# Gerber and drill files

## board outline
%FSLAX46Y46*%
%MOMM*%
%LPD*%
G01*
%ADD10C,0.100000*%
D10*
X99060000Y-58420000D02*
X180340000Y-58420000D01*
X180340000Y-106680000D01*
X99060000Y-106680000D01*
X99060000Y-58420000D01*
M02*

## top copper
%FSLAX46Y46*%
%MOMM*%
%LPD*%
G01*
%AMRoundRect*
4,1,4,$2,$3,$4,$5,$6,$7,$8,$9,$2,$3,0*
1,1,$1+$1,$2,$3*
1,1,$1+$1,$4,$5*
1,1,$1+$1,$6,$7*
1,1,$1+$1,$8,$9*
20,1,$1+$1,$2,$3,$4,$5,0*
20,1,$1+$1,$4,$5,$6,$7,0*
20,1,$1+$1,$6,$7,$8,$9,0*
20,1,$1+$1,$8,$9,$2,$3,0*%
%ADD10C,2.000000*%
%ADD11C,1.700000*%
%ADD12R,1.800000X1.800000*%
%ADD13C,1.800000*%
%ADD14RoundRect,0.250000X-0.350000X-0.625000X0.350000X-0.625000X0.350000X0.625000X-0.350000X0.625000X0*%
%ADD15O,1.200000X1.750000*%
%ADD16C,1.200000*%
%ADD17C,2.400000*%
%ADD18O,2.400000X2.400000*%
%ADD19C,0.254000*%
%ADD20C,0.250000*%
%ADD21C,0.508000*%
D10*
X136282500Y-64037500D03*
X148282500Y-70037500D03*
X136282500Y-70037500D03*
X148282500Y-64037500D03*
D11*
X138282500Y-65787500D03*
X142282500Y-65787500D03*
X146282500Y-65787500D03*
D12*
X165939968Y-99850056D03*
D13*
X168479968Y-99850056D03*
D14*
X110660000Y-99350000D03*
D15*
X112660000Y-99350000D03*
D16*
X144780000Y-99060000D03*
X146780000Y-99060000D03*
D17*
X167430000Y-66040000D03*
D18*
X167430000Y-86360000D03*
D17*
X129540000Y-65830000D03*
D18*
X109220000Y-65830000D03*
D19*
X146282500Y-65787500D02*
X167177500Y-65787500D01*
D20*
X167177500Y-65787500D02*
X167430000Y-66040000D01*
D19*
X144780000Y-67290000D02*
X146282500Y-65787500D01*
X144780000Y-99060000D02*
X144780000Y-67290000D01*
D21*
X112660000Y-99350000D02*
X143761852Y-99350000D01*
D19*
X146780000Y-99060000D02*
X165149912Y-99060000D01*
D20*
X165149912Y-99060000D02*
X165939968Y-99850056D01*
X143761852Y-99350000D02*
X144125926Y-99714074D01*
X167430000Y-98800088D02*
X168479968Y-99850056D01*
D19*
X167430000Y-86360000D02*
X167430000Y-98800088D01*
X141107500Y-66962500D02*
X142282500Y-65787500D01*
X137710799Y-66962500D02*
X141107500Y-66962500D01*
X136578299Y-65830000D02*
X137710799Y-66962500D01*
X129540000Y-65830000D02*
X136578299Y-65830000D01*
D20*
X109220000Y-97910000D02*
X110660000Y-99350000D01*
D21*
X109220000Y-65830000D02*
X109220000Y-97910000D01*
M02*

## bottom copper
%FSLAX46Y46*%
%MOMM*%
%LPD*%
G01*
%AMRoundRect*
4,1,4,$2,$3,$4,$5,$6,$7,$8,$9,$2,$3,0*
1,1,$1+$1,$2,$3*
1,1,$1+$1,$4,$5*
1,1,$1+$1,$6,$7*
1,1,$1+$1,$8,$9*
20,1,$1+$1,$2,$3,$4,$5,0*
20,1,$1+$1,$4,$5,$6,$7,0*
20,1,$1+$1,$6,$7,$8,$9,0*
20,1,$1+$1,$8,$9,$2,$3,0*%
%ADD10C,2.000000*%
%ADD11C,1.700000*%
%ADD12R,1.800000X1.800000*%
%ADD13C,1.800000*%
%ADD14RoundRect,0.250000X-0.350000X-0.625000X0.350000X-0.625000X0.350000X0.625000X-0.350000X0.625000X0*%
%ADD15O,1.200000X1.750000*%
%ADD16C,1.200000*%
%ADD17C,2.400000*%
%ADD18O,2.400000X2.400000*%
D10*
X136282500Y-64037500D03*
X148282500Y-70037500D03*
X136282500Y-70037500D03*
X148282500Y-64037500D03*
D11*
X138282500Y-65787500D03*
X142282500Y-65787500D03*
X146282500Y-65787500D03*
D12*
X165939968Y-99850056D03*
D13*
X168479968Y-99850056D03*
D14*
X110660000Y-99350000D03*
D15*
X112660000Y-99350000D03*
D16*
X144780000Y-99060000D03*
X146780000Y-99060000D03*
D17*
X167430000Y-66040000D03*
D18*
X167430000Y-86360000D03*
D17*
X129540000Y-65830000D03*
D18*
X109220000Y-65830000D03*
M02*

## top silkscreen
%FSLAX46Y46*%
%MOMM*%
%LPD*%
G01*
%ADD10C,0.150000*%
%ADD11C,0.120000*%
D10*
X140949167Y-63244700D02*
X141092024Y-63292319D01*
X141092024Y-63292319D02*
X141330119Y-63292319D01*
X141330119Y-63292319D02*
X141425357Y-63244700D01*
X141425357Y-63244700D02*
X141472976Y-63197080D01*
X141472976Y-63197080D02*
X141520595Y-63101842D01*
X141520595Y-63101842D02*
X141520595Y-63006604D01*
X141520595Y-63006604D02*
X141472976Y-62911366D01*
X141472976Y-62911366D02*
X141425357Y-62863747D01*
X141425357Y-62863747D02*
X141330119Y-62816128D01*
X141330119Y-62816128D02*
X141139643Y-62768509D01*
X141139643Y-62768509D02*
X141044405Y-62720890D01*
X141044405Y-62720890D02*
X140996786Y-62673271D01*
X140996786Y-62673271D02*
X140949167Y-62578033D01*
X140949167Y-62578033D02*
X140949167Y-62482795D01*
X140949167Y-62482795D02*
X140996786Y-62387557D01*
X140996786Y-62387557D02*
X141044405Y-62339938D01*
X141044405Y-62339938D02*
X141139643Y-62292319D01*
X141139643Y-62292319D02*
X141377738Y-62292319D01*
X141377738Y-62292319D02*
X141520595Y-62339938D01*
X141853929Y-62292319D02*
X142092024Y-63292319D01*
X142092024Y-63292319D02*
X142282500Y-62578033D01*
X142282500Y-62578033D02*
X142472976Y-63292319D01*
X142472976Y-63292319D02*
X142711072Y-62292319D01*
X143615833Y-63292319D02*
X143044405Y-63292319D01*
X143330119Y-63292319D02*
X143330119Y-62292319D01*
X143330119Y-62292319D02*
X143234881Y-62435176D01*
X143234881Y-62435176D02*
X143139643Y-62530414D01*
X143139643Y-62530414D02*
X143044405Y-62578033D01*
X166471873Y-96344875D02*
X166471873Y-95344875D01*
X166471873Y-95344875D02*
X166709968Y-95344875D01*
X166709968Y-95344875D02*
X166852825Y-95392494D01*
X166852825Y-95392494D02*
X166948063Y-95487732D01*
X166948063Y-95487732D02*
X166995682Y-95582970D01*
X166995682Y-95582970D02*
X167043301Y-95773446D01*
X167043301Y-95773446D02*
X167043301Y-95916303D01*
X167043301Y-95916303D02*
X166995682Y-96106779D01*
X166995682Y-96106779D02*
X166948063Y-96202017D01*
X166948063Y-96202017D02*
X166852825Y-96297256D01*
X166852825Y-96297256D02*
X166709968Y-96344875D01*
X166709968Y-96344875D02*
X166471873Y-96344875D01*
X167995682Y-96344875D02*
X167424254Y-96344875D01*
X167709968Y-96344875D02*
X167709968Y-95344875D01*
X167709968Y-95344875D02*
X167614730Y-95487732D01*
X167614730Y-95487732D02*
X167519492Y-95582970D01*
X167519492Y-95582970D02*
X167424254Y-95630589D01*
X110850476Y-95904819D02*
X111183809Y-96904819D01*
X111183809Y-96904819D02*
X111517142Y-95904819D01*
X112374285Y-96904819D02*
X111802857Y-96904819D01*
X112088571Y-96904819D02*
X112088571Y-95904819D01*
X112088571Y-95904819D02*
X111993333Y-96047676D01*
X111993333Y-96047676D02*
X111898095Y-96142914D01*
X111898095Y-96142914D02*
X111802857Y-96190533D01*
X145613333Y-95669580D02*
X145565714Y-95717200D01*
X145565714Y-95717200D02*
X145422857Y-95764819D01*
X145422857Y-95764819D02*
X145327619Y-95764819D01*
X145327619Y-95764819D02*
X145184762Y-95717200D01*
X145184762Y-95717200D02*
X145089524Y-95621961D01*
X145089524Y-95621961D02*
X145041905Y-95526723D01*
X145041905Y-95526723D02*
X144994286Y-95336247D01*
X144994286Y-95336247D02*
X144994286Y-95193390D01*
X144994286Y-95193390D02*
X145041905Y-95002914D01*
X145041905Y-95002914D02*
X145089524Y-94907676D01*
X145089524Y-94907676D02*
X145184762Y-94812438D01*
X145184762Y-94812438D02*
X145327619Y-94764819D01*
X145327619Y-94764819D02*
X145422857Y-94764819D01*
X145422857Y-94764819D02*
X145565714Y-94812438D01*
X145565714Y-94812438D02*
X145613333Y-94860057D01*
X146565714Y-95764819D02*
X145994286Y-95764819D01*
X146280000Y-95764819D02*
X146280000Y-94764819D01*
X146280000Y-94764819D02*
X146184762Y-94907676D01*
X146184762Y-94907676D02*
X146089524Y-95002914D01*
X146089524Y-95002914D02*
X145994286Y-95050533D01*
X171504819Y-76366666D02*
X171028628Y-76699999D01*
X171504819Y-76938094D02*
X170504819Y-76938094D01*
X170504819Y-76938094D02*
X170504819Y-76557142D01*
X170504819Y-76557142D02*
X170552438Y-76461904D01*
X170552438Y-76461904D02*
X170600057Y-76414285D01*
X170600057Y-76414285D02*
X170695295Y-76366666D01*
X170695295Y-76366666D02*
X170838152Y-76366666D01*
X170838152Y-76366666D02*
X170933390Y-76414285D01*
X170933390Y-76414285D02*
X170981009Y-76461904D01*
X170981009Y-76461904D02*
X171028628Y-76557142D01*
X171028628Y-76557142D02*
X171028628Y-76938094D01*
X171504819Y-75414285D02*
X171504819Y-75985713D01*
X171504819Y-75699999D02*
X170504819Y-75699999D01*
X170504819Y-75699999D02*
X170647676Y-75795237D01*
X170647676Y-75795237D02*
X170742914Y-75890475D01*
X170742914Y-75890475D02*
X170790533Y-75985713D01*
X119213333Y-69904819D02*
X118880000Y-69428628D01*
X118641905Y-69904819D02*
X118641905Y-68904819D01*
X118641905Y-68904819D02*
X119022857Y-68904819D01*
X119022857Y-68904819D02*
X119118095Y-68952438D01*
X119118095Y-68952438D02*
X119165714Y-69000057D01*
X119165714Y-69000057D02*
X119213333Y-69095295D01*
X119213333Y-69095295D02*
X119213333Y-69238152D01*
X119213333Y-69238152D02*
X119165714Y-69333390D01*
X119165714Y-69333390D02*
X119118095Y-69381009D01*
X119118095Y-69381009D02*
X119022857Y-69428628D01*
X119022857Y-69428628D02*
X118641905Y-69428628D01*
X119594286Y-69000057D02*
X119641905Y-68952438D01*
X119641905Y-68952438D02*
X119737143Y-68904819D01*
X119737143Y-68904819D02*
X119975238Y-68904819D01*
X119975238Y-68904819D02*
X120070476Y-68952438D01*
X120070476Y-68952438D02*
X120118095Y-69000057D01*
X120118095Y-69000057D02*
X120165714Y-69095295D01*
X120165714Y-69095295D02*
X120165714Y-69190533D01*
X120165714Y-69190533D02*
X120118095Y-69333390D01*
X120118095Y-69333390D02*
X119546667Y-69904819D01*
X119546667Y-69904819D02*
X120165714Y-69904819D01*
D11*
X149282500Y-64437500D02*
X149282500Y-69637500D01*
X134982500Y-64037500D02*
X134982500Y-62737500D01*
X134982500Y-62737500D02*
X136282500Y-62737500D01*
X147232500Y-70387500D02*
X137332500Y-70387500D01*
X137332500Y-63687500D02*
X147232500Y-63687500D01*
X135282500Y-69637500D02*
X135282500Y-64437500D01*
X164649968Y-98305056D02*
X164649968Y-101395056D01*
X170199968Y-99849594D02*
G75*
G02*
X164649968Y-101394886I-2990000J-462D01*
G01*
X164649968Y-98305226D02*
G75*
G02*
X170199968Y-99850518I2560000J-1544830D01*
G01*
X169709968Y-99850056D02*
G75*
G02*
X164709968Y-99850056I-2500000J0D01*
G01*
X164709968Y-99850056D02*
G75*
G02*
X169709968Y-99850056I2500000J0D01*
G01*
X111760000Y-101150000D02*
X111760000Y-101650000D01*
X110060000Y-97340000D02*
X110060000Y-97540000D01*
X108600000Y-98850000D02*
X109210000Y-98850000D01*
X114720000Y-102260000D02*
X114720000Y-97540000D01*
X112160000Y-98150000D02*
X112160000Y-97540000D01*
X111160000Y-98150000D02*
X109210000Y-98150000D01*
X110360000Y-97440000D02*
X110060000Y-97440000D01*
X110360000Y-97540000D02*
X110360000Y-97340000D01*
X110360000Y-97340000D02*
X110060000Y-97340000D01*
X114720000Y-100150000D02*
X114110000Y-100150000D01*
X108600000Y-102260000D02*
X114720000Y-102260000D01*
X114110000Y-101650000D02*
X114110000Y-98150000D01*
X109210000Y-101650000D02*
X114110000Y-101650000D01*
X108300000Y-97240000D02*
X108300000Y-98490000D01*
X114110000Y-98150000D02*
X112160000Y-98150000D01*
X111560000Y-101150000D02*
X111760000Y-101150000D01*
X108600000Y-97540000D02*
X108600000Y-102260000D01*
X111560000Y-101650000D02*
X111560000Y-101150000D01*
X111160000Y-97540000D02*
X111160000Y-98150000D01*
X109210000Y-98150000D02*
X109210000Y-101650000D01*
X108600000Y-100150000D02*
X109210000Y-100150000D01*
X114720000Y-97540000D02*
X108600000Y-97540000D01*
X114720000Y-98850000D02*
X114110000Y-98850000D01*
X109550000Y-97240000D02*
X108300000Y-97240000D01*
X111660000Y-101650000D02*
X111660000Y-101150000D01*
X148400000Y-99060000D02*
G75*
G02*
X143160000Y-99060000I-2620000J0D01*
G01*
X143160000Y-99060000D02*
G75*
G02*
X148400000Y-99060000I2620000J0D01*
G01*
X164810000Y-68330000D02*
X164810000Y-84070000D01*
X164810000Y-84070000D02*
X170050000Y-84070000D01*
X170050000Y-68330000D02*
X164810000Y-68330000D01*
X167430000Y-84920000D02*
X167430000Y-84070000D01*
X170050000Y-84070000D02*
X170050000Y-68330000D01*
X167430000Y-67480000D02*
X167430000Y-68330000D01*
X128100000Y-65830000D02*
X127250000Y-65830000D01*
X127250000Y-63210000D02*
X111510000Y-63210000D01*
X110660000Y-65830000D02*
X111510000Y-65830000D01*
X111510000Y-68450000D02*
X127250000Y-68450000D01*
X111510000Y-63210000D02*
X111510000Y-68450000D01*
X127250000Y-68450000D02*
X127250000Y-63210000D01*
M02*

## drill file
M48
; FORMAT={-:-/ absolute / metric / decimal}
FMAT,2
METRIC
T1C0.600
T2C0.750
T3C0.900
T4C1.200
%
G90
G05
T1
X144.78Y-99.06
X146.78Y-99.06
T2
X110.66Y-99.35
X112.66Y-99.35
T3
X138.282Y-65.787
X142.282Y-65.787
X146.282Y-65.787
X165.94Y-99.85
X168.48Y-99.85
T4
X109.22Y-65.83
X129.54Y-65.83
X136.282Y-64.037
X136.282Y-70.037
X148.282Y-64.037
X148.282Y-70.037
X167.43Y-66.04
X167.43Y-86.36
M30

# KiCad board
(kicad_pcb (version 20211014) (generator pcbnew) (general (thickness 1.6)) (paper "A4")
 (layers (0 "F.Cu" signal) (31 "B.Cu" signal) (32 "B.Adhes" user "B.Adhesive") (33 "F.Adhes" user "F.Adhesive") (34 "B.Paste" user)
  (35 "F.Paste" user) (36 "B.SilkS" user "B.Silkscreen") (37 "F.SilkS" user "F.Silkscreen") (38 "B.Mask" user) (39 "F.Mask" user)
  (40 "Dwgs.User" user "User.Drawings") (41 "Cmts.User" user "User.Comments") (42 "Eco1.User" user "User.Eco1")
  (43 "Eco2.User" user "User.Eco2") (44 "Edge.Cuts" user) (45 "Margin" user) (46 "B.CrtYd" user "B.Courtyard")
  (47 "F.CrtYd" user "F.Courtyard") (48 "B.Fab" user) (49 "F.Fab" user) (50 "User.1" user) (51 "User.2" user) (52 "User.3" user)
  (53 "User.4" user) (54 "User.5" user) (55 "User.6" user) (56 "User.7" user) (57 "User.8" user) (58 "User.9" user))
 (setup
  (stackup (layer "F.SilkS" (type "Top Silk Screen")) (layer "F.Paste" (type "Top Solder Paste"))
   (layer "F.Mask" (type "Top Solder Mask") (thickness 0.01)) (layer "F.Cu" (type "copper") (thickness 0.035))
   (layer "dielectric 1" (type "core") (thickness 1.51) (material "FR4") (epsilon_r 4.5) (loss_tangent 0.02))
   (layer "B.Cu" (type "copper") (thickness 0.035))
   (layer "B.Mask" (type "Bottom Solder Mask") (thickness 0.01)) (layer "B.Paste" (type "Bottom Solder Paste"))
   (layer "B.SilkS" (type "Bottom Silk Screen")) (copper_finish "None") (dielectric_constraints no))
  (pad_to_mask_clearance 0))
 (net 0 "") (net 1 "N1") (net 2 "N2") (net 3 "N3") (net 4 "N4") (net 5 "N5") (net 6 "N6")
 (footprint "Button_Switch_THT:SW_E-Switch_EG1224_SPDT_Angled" (layer "F.Cu") (at 138.2825 65.7875)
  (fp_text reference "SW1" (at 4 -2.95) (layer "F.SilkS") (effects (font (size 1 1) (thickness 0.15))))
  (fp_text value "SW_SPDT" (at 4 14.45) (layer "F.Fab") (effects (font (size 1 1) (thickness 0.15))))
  (fp_line (start 11 -1.35) (end 11 3.85) (layer "F.SilkS") (width 0.12))
  (fp_line (start -3.3 -1.75) (end -3.3 -3.05) (layer "F.SilkS") (width 0.12))
  (fp_line (start -3.3 -3.05) (end -2 -3.05) (layer "F.SilkS") (width 0.12))
  (fp_line (start 8.95 4.6) (end -0.95 4.6) (layer "F.SilkS") (width 0.12))
  (fp_line (start -0.95 -2.1) (end 8.95 -2.1) (layer "F.SilkS") (width 0.12))
  (fp_line (start -3 3.85) (end -3 -1.35) (layer "F.SilkS") (width 0.12))
  (pad "" thru_hole circle (at -2 -1.75) (size 2 2) (drill 1.2) (layers *.Cu *.Mask))
  (pad "" thru_hole circle (at 10 4.25) (size 2 2) (drill 1.2) (layers *.Cu *.Mask))
  (pad "" thru_hole circle (at -2 4.25) (size 2 2) (drill 1.2) (layers *.Cu *.Mask))
  (pad "" thru_hole circle (at 10 -1.75) (size 2 2) (drill 1.2) (layers *.Cu *.Mask))
  (pad "1" thru_hole circle (at 0 0) (size 1.7 1.7) (drill 0.9) (layers *.Cu *.Mask) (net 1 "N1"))
  (pad "2" thru_hole circle (at 4 0) (size 1.7 1.7) (drill 0.9) (layers *.Cu *.Mask) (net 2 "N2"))
  (pad "3" thru_hole circle (at 8 0) (size 1.7 1.7) (drill 0.9) (layers *.Cu *.Mask) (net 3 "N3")))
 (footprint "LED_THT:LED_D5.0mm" (layer "F.Cu") (at 165.939968 99.850056)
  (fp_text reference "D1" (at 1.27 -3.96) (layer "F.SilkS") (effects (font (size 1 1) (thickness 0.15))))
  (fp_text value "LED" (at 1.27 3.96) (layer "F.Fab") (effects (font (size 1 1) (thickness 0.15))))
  (fp_line (start -1.29 -1.545) (end -1.29 1.545) (layer "F.SilkS") (width 0.12))
  (fp_arc (start 4.26 -0.000462) (mid 2.072002 2.880433) (end -1.29 1.54483) (layer "F.SilkS") (width 0.12))
  (fp_arc (start -1.29 -1.54483) (mid 2.072002 -2.880433) (end 4.26 0.000462) (layer "F.SilkS") (width 0.12))
  (fp_circle (center 1.27 0) (end 3.77 0) (layer "F.SilkS") (width 0.12) (fill none))
  (pad "1" thru_hole rect (at 0 0) (size 1.8 1.8) (drill 0.9) (layers *.Cu *.Mask) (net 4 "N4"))
  (pad "2" thru_hole circle (at 2.54 0) (size 1.8 1.8) (drill 0.9) (layers *.Cu *.Mask) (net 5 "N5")))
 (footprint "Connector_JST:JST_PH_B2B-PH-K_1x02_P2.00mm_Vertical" (layer "F.Cu") (at 110.66 99.35)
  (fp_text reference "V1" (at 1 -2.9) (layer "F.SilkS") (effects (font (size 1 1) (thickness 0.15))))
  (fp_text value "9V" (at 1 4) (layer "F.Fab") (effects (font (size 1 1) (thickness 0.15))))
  (fp_line (start 1.1 1.8) (end 1.1 2.3) (layer "F.SilkS") (width 0.12))
  (fp_line (start -0.6 -2.01) (end -0.6 -1.81) (layer "F.SilkS") (width 0.12))
  (fp_line (start -2.06 -0.5) (end -1.45 -0.5) (layer "F.SilkS") (width 0.12))
  (fp_line (start 4.06 2.91) (end 4.06 -1.81) (layer "F.SilkS") (width 0.12))
  (fp_line (start 1.5 -1.2) (end 1.5 -1.81) (layer "F.SilkS") (width 0.12))
  (fp_line (start 0.5 -1.2) (end -1.45 -1.2) (layer "F.SilkS") (width 0.12))
  (fp_line (start -0.3 -1.91) (end -0.6 -1.91) (layer "F.SilkS") (width 0.12))
  (fp_line (start -0.3 -1.81) (end -0.3 -2.01) (layer "F.SilkS") (width 0.12))
  (fp_line (start -0.3 -2.01) (end -0.6 -2.01) (layer "F.SilkS") (width 0.12))
  (fp_line (start 4.06 0.8) (end 3.45 0.8) (layer "F.SilkS") (width 0.12))
  (fp_line (start -2.06 2.91) (end 4.06 2.91) (layer "F.SilkS") (width 0.12))
  (fp_line (start 3.45 2.3) (end 3.45 -1.2) (layer "F.SilkS") (width 0.12))
  (fp_line (start -1.45 2.3) (end 3.45 2.3) (layer "F.SilkS") (width 0.12))
  (fp_line (start -2.36 -2.11) (end -2.36 -0.86) (layer "F.SilkS") (width 0.12))
  (fp_line (start 3.45 -1.2) (end 1.5 -1.2) (layer "F.SilkS") (width 0.12))
  (fp_line (start 0.9 1.8) (end 1.1 1.8) (layer "F.SilkS") (width 0.12))
  (fp_line (start -2.06 -1.81) (end -2.06 2.91) (layer "F.SilkS") (width 0.12))
  (fp_line (start 0.9 2.3) (end 0.9 1.8) (layer "F.SilkS") (width 0.12))
  (fp_line (start 0.5 -1.81) (end 0.5 -1.2) (layer "F.SilkS") (width 0.12))
  (fp_line (start -1.45 -1.2) (end -1.45 2.3) (layer "F.SilkS") (width 0.12))
  (fp_line (start -2.06 0.8) (end -1.45 0.8) (layer "F.SilkS") (width 0.12))
  (fp_line (start 4.06 -1.81) (end -2.06 -1.81) (layer "F.SilkS") (width 0.12))
  (fp_line (start 4.06 -0.5) (end 3.45 -0.5) (layer "F.SilkS") (width 0.12))
  (fp_line (start -1.11 -2.11) (end -2.36 -2.11) (layer "F.SilkS") (width 0.12))
  (fp_line (start 1 2.3) (end 1 1.8) (layer "F.SilkS") (width 0.12))
  (pad "1" thru_hole roundrect (at 0 0) (size 1.2 1.75) (drill 0.75) (layers *.Cu *.Mask) (roundrect_rratio 0.208333) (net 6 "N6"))
  (pad "2" thru_hole oval (at 2 0) (size 1.2 1.75) (drill 0.75) (layers *.Cu *.Mask) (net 4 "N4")))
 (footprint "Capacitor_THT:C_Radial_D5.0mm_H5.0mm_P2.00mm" (layer "F.Cu") (at 144.78 99.06)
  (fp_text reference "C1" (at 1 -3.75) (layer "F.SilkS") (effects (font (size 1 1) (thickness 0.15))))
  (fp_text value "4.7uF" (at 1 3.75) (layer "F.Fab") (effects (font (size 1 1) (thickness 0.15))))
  (fp_circle (center 1 0) (end 3.62 0) (layer "F.SilkS") (width 0.12) (fill none))
  (pad "1" thru_hole circle (at 0 0) (size 1.2 1.2) (drill 0.6) (layers *.Cu *.Mask) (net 3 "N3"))
  (pad "2" thru_hole circle (at 2 0) (size 1.2 1.2) (drill 0.6) (layers *.Cu *.Mask) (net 4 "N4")))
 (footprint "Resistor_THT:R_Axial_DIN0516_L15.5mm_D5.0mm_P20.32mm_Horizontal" (layer "F.Cu") (at 167.43 66.04 -90)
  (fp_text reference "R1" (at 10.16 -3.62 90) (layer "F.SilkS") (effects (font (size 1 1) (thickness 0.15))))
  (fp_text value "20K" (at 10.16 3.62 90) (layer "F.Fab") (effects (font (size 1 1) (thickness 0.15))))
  (fp_line (start 2.29 2.62) (end 18.03 2.62) (layer "F.SilkS") (width 0.12))
  (fp_line (start 18.03 2.62) (end 18.03 -2.62) (layer "F.SilkS") (width 0.12))
  (fp_line (start 2.29 -2.62) (end 2.29 2.62) (layer "F.SilkS") (width 0.12))
  (fp_line (start 18.88 0) (end 18.03 0) (layer "F.SilkS") (width 0.12))
  (fp_line (start 18.03 -2.62) (end 2.29 -2.62) (layer "F.SilkS") (width 0.12))
  (fp_line (start 1.44 0) (end 2.29 0) (layer "F.SilkS") (width 0.12))
  (pad "1" thru_hole circle (at 0 0 270) (size 2.4 2.4) (drill 1.2) (layers *.Cu *.Mask) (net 3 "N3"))
  (pad "2" thru_hole oval (at 20.32 0 270) (size 2.4 2.4) (drill 1.2) (layers *.Cu *.Mask) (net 5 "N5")))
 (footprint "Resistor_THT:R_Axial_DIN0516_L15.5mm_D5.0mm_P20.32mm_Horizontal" (layer "F.Cu") (at 129.54 65.83 180)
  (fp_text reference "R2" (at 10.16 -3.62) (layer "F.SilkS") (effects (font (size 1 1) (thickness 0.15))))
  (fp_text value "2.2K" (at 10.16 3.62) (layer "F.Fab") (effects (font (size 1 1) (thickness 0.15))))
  (fp_line (start 1.44 0) (end 2.29 0) (layer "F.SilkS") (width 0.12))
  (fp_line (start 2.29 2.62) (end 18.03 2.62) (layer "F.SilkS") (width 0.12))
  (fp_line (start 18.88 0) (end 18.03 0) (layer "F.SilkS") (width 0.12))
  (fp_line (start 18.03 -2.62) (end 2.29 -2.62) (layer "F.SilkS") (width 0.12))
  (fp_line (start 18.03 2.62) (end 18.03 -2.62) (layer "F.SilkS") (width 0.12))
  (fp_line (start 2.29 -2.62) (end 2.29 2.62) (layer "F.SilkS") (width 0.12))
  (pad "1" thru_hole circle (at 0 0 180) (size 2.4 2.4) (drill 1.2) (layers *.Cu *.Mask) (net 2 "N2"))
  (pad "2" thru_hole oval (at 20.32 0 180) (size 2.4 2.4) (drill 1.2) (layers *.Cu *.Mask) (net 6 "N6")))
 (gr_rect (start 180.34 106.68) (end 99.06 58.42) (layer "Edge.Cuts") (width 0.1) (fill none))
 (segment (start 146.2825 65.7875) (end 167.1775 65.7875) (width 0.254) (layer "F.Cu") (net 3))
 (segment (start 167.1775 65.7875) (end 167.43 66.04) (width 0.25) (layer "F.Cu") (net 3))
 (segment (start 144.78 67.29) (end 146.2825 65.7875) (width 0.254) (layer "F.Cu") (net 3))
 (segment (start 144.78 99.06) (end 144.78 67.29) (width 0.254) (layer "F.Cu") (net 3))
 (segment (start 112.66 99.35) (end 143.761852 99.35) (width 0.508) (layer "F.Cu") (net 4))
 (segment (start 146.78 99.06) (end 165.149912 99.06) (width 0.254) (layer "F.Cu") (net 4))
 (segment (start 165.149912 99.06) (end 165.939968 99.850056) (width 0.25) (layer "F.Cu") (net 4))
 (segment (start 143.761852 99.35) (end 144.125926 99.714074) (width 0.25) (layer "F.Cu") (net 4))
 (segment (start 167.43 98.800088) (end 168.479968 99.850056) (width 0.25) (layer "F.Cu") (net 5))
 (segment (start 167.43 86.36) (end 167.43 98.800088) (width 0.254) (layer "F.Cu") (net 5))
 (segment (start 141.1075 66.9625) (end 142.2825 65.7875) (width 0.254) (layer "F.Cu") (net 2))
 (segment (start 137.710799 66.9625) (end 141.1075 66.9625) (width 0.254) (layer "F.Cu") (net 2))
 (segment (start 136.578299 65.83) (end 137.710799 66.9625) (width 0.254) (layer "F.Cu") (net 2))
 (segment (start 129.54 65.83) (end 136.578299 65.83) (width 0.254) (layer "F.Cu") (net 2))
 (segment (start 109.22 97.91) (end 110.66 99.35) (width 0.25) (layer "F.Cu") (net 6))
 (segment (start 109.22 65.83) (end 109.22 97.91) (width 0.508) (layer "F.Cu") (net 6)))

